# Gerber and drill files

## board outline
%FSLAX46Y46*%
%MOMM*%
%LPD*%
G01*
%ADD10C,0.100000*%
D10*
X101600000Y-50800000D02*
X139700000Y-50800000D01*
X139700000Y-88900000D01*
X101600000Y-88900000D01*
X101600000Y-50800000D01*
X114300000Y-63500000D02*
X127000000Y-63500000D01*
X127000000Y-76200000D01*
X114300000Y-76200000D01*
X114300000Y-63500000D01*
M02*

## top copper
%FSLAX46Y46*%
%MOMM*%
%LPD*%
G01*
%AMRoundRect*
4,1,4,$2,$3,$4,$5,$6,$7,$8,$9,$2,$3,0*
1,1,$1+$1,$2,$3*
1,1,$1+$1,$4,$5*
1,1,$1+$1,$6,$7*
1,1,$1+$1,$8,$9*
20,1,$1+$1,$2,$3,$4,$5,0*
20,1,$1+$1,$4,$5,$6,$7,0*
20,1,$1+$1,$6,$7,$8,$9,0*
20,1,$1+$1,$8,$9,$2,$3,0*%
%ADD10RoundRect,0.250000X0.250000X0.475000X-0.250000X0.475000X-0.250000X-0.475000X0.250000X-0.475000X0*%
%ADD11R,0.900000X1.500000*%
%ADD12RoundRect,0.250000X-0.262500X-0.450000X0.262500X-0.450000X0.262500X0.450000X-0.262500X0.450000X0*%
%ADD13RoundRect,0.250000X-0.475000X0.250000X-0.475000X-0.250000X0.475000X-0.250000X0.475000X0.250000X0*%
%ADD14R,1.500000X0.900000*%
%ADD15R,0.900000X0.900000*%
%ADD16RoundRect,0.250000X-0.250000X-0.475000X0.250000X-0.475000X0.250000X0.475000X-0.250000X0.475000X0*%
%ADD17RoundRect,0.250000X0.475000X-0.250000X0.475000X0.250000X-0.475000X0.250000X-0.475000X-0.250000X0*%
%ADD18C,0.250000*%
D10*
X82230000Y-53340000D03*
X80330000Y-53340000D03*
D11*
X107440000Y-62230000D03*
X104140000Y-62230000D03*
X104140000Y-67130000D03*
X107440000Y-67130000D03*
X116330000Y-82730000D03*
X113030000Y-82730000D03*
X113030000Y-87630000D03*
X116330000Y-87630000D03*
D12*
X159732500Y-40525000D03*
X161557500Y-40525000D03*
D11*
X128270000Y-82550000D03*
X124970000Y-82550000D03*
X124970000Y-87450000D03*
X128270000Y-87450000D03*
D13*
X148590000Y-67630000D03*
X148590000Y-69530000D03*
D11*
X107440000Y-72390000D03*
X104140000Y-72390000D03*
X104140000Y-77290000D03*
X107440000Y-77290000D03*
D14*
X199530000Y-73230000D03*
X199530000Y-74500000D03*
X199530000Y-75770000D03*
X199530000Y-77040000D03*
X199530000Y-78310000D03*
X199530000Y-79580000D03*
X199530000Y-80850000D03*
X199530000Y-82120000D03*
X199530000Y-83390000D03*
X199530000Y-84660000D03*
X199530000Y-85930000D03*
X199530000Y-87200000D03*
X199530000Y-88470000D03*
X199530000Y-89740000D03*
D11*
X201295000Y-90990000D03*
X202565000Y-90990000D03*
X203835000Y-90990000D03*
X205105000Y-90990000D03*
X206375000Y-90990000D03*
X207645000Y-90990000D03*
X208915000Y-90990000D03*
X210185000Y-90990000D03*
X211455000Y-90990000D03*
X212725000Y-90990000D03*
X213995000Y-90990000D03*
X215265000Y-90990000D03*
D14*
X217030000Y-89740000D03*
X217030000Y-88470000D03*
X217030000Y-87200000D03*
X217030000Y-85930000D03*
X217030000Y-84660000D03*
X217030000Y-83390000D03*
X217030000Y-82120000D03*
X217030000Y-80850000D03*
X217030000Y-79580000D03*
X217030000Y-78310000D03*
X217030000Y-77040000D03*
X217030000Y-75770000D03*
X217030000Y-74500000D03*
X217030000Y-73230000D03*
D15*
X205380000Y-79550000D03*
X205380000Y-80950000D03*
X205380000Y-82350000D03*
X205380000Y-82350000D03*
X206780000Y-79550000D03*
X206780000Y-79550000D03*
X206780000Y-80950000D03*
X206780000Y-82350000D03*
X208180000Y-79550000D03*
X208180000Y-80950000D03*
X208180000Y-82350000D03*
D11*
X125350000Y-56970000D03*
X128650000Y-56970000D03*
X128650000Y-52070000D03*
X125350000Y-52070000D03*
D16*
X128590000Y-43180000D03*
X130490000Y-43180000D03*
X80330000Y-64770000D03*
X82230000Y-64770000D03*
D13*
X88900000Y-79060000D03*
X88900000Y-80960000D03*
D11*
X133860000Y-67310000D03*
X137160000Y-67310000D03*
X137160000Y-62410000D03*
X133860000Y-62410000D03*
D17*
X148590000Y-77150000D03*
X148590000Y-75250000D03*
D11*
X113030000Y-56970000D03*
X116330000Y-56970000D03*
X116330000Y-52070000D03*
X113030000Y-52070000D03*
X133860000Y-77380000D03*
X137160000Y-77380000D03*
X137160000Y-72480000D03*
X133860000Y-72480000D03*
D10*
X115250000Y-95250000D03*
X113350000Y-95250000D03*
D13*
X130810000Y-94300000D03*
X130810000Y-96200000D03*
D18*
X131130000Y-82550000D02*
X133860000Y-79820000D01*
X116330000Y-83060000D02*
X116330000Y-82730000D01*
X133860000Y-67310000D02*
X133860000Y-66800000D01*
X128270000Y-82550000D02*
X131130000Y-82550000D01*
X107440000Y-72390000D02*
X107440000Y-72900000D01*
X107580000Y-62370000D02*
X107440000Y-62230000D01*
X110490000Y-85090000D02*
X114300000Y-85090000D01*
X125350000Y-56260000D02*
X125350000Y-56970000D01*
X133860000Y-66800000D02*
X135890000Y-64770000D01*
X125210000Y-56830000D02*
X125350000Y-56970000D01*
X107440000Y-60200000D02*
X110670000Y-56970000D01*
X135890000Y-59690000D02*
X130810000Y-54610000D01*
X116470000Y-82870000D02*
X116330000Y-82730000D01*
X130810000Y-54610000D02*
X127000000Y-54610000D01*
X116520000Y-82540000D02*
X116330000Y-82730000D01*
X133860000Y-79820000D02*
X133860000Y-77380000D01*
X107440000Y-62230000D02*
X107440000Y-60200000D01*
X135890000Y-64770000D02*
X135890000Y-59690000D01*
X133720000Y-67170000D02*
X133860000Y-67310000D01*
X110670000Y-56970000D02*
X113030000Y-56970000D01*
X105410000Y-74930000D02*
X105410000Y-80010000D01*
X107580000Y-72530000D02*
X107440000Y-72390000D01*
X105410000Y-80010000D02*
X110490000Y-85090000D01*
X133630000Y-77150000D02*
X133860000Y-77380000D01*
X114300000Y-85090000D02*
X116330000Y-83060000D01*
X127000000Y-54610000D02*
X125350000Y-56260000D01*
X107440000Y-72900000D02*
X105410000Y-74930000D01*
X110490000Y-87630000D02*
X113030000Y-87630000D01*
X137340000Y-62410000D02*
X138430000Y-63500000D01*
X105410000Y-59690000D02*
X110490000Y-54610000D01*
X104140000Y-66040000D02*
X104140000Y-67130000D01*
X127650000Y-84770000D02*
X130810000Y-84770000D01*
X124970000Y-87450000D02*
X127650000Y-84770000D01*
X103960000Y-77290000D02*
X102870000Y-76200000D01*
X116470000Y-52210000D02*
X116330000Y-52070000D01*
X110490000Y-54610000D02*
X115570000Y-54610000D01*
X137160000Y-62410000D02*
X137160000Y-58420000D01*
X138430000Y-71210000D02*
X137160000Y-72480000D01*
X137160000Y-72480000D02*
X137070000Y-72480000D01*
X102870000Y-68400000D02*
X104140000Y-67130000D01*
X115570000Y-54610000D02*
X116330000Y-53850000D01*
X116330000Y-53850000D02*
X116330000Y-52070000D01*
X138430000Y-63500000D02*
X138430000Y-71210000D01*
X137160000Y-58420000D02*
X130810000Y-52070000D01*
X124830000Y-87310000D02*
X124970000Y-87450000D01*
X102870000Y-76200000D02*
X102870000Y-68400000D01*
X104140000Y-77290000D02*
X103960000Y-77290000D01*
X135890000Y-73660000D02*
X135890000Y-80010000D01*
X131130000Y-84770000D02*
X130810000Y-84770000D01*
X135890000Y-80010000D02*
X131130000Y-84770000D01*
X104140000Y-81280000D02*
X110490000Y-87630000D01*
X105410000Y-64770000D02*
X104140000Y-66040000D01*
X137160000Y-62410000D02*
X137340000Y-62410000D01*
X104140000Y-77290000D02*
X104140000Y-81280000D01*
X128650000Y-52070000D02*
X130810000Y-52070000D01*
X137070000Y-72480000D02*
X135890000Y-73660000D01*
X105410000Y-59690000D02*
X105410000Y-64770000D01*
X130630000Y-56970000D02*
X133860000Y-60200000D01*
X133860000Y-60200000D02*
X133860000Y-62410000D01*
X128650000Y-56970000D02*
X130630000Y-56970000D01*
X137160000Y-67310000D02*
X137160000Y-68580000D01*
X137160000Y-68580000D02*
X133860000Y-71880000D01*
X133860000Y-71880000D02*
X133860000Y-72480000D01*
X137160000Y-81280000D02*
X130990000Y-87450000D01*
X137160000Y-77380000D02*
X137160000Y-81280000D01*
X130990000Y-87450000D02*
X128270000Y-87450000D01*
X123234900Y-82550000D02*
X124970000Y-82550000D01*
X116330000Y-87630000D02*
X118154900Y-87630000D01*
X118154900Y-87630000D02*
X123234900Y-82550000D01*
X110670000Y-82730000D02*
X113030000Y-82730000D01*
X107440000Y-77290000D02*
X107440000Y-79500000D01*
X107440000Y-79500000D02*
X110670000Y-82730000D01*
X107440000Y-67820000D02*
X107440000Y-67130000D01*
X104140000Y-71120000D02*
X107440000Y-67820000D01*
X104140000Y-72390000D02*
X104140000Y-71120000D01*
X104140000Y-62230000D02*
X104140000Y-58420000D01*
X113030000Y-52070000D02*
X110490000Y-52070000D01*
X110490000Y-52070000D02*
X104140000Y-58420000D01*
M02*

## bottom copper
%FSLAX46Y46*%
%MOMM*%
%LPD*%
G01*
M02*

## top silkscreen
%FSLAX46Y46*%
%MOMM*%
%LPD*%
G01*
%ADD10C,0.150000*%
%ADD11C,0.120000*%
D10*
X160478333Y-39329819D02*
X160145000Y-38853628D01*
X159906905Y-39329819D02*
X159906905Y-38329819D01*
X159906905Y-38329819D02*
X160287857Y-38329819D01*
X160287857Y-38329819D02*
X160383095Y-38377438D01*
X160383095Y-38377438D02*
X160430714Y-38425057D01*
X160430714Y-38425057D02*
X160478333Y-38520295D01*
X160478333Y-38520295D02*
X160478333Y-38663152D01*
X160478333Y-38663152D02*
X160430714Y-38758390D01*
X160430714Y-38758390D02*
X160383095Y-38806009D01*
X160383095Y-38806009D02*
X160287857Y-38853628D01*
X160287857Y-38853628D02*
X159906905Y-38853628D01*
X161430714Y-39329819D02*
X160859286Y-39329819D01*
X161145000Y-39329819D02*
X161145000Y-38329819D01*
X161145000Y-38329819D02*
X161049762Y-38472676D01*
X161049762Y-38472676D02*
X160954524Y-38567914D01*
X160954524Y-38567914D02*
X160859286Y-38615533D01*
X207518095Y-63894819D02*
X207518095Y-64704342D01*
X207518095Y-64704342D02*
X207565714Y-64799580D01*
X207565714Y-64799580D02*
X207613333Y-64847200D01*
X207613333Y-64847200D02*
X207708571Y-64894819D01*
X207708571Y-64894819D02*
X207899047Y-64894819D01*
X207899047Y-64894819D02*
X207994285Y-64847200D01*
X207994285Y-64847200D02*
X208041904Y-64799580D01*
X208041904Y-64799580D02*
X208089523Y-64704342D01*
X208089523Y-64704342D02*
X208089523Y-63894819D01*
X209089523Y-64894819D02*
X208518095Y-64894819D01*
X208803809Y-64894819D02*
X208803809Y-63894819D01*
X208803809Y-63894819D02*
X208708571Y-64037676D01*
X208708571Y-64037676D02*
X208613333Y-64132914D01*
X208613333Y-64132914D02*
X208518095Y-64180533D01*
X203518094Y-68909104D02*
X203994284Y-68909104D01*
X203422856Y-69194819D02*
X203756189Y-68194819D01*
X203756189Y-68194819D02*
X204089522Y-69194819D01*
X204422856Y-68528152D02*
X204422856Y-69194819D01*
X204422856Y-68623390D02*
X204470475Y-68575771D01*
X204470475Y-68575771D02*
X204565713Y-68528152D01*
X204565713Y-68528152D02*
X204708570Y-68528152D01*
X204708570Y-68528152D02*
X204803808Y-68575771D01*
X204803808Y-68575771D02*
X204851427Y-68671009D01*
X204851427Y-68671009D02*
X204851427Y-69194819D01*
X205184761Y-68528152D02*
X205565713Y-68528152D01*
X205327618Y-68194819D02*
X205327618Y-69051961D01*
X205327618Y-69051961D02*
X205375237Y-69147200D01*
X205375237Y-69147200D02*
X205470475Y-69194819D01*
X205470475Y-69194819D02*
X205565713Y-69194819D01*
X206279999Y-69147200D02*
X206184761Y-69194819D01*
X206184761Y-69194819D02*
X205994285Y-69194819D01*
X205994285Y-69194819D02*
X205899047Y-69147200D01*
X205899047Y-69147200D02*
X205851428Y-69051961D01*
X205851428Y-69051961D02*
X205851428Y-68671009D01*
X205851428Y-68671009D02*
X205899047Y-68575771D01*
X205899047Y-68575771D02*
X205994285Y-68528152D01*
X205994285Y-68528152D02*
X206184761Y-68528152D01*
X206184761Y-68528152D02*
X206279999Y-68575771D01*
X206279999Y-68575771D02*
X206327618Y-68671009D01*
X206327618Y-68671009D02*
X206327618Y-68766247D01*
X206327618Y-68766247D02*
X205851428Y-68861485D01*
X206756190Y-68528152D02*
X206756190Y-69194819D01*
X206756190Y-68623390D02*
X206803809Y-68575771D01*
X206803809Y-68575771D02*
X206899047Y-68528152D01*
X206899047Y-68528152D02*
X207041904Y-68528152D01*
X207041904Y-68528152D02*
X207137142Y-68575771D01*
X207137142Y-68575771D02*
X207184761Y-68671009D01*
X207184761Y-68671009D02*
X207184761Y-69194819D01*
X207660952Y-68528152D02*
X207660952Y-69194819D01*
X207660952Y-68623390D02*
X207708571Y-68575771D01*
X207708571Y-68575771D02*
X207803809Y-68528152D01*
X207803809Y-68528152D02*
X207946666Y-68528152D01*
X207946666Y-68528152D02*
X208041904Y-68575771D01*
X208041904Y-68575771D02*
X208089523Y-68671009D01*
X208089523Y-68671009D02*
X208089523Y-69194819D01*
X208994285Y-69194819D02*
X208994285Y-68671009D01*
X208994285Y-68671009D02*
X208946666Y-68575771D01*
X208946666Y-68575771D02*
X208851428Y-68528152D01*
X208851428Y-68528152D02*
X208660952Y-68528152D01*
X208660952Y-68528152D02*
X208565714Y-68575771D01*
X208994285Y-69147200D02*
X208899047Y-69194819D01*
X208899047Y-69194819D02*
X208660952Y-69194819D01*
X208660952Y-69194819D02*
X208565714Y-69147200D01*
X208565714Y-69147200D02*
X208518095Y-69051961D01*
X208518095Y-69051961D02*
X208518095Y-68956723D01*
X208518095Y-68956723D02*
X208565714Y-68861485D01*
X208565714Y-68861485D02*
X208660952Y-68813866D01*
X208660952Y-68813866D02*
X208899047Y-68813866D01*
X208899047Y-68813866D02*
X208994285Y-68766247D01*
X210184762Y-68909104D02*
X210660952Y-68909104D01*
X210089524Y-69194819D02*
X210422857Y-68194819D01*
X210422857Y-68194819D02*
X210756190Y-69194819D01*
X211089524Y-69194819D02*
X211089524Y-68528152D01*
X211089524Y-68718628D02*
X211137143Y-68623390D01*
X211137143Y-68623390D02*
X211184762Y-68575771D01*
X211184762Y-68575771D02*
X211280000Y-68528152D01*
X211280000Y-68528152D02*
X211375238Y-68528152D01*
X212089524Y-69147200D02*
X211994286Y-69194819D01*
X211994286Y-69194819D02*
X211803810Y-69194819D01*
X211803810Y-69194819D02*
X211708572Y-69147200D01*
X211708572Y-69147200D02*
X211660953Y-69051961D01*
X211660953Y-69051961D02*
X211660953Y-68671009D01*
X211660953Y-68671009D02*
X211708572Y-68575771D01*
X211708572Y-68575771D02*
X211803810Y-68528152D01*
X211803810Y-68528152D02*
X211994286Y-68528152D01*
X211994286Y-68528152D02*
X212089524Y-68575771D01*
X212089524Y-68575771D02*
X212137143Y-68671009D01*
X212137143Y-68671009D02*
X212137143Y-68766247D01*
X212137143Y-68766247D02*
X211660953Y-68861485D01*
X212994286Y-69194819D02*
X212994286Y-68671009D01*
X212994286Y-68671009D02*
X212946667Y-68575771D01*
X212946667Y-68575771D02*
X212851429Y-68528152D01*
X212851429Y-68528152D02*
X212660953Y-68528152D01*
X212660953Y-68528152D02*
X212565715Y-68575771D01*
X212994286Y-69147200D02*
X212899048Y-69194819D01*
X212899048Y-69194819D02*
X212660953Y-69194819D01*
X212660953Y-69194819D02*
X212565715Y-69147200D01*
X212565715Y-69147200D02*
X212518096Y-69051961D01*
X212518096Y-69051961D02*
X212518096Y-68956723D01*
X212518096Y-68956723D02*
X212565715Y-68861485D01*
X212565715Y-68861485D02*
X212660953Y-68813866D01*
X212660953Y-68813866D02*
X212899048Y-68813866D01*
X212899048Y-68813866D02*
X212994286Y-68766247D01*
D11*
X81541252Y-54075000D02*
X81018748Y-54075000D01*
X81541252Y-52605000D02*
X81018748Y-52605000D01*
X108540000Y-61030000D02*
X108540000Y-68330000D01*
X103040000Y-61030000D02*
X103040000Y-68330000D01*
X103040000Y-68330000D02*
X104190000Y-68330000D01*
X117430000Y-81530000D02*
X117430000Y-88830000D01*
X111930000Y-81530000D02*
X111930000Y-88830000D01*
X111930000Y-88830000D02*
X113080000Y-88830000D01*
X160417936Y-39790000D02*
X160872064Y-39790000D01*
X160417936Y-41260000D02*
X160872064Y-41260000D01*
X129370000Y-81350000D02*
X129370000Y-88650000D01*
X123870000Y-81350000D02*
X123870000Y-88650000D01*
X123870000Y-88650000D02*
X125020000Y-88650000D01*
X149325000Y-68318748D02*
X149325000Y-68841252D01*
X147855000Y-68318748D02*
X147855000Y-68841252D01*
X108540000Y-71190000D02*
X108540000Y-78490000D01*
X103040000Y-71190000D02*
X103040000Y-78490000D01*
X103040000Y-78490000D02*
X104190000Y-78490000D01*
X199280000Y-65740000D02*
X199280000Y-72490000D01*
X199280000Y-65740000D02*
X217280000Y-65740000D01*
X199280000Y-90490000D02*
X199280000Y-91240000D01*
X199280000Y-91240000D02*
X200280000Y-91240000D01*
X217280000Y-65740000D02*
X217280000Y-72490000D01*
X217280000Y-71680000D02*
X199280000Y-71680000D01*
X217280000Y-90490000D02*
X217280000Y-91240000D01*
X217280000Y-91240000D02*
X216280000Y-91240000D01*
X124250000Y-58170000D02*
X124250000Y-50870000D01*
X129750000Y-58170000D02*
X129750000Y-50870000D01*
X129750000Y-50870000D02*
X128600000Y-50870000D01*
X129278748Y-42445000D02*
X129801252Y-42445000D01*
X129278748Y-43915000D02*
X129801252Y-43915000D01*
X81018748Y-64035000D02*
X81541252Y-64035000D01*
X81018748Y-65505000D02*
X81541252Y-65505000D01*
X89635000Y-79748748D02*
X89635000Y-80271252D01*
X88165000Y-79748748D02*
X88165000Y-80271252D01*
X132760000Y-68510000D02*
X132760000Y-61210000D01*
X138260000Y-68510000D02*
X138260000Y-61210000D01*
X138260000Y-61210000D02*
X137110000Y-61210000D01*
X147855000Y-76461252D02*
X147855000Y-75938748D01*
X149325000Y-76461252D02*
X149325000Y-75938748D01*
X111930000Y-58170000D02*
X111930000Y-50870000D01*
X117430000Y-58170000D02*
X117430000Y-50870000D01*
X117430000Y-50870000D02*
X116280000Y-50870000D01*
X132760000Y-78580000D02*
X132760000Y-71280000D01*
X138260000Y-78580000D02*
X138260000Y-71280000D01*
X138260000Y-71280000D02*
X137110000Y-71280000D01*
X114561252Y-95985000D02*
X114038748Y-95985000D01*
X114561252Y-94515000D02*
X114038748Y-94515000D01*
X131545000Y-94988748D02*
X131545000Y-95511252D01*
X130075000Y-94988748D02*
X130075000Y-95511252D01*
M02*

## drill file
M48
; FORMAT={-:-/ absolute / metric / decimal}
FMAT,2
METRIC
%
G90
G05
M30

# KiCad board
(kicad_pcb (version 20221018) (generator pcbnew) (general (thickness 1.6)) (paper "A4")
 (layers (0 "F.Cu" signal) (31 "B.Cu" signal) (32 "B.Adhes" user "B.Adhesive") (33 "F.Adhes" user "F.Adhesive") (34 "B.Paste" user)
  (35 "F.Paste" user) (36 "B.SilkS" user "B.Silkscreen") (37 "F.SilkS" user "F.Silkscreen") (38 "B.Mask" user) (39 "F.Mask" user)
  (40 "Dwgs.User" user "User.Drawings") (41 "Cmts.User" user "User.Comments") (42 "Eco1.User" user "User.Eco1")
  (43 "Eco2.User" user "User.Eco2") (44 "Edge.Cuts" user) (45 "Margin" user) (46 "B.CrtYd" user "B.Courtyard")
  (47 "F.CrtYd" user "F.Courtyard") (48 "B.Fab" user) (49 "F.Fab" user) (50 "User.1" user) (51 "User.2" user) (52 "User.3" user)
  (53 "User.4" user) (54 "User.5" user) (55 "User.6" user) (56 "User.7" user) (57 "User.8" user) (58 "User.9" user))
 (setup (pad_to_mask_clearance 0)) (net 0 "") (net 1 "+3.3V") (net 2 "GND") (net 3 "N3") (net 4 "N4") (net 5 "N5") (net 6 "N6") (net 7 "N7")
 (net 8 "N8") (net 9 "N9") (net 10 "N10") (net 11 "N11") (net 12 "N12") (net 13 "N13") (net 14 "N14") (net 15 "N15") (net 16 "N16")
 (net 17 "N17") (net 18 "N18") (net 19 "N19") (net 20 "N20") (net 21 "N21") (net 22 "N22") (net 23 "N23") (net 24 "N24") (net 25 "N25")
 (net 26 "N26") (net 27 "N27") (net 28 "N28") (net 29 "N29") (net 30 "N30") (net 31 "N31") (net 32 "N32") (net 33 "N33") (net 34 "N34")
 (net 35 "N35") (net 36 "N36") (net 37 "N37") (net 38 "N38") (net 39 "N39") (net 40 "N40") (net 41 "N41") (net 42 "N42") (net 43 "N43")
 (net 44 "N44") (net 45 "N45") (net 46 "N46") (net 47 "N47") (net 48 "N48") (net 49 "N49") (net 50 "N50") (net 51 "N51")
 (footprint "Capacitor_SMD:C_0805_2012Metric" (layer "F.Cu") (at 81.28 53.34 180)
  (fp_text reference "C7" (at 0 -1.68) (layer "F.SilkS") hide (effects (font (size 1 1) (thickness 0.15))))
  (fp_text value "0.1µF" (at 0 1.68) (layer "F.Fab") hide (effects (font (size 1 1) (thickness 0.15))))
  (fp_line (start -0.261252 -0.735) (end 0.261252 -0.735) (stroke (width 0.12) (type solid)) (layer "F.SilkS"))
  (fp_line (start -0.261252 0.735) (end 0.261252 0.735) (stroke (width 0.12) (type solid)) (layer "F.SilkS"))
  (pad "1" smd roundrect (at -0.95 0 180) (size 1 1.45) (layers "F.Cu" "F.Paste" "F.Mask") (roundrect_rratio 0.25) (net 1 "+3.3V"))
  (pad "2" smd roundrect (at 0.95 0 180) (size 1 1.45) (layers "F.Cu" "F.Paste" "F.Mask") (roundrect_rratio 0.25) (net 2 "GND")))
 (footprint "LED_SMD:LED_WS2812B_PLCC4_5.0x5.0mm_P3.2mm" (layer "F.Cu") (at 105.79 64.68 -90)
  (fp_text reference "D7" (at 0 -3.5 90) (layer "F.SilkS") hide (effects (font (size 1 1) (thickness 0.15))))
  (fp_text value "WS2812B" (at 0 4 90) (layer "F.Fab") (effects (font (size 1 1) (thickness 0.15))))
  (fp_line (start -3.65 -2.75) (end 3.65 -2.75) (stroke (width 0.12) (type solid)) (layer "F.SilkS"))
  (fp_line (start -3.65 2.75) (end 3.65 2.75) (stroke (width 0.12) (type solid)) (layer "F.SilkS"))
  (fp_line (start 3.65 2.75) (end 3.65 1.6) (stroke (width 0.12) (type solid)) (layer "F.SilkS"))
  (pad "1" smd rect (at -2.45 -1.65 270) (size 1.5 0.9) (layers "F.Cu" "F.Paste" "F.Mask") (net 1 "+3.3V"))
  (pad "2" smd rect (at -2.45 1.65 270) (size 1.5 0.9) (layers "F.Cu" "F.Paste" "F.Mask") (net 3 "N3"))
  (pad "3" smd rect (at 2.45 1.65 270) (size 1.5 0.9) (layers "F.Cu" "F.Paste" "F.Mask") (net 2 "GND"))
  (pad "4" smd rect (at 2.45 -1.65 270) (size 1.5 0.9) (layers "F.Cu" "F.Paste" "F.Mask") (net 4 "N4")))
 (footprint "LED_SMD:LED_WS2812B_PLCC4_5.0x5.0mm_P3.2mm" (layer "F.Cu") (at 114.68 85.18 -90)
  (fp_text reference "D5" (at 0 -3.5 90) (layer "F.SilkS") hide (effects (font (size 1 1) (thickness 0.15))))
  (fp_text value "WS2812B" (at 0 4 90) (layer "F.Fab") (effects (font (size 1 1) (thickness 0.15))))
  (fp_line (start -3.65 -2.75) (end 3.65 -2.75) (stroke (width 0.12) (type solid)) (layer "F.SilkS"))
  (fp_line (start -3.65 2.75) (end 3.65 2.75) (stroke (width 0.12) (type solid)) (layer "F.SilkS"))
  (fp_line (start 3.65 2.75) (end 3.65 1.6) (stroke (width 0.12) (type solid)) (layer "F.SilkS"))
  (pad "1" smd rect (at -2.45 -1.65 270) (size 1.5 0.9) (layers "F.Cu" "F.Paste" "F.Mask") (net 1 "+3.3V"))
  (pad "2" smd rect (at -2.45 1.65 270) (size 1.5 0.9) (layers "F.Cu" "F.Paste" "F.Mask") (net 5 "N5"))
  (pad "3" smd rect (at 2.45 1.65 270) (size 1.5 0.9) (layers "F.Cu" "F.Paste" "F.Mask") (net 2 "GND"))
  (pad "4" smd rect (at 2.45 -1.65 270) (size 1.5 0.9) (layers "F.Cu" "F.Paste" "F.Mask") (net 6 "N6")))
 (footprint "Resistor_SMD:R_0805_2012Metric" (layer "F.Cu") (at 160.645 40.525)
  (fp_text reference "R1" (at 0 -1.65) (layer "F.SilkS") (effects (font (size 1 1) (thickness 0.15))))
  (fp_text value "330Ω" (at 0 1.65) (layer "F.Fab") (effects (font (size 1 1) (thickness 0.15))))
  (fp_line (start -0.227064 -0.735) (end 0.227064 -0.735) (stroke (width 0.12) (type solid)) (layer "F.SilkS"))
  (fp_line (start -0.227064 0.735) (end 0.227064 0.735) (stroke (width 0.12) (type solid)) (layer "F.SilkS"))
  (pad "1" smd roundrect (at -0.9125 0) (size 1.025 1.4) (layers "F.Cu" "F.Paste" "F.Mask") (roundrect_rratio 0.243902) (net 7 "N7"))
  (pad "2" smd roundrect (at 0.9125 0) (size 1.025 1.4) (layers "F.Cu" "F.Paste" "F.Mask") (roundrect_rratio 0.243902) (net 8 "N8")))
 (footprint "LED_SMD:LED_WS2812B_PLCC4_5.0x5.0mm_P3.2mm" (layer "F.Cu") (at 126.62 85 -90)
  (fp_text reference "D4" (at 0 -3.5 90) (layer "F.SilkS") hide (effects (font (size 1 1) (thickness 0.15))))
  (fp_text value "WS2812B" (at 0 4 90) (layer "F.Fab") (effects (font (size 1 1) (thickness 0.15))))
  (fp_line (start -3.65 -2.75) (end 3.65 -2.75) (stroke (width 0.12) (type solid)) (layer "F.SilkS"))
  (fp_line (start -3.65 2.75) (end 3.65 2.75) (stroke (width 0.12) (type solid)) (layer "F.SilkS"))
  (fp_line (start 3.65 2.75) (end 3.65 1.6) (stroke (width 0.12) (type solid)) (layer "F.SilkS"))
  (pad "1" smd rect (at -2.45 -1.65 270) (size 1.5 0.9) (layers "F.Cu" "F.Paste" "F.Mask") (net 1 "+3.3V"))
  (pad "2" smd rect (at -2.45 1.65 270) (size 1.5 0.9) (layers "F.Cu" "F.Paste" "F.Mask") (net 6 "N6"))
  (pad "3" smd rect (at 2.45 1.65 270) (size 1.5 0.9) (layers "F.Cu" "F.Paste" "F.Mask") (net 2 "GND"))
  (pad "4" smd rect (at 2.45 -1.65 270) (size 1.5 0.9) (layers "F.Cu" "F.Paste" "F.Mask") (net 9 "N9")))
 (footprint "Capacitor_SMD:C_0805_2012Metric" (layer "F.Cu") (at 148.59 68.58 -90)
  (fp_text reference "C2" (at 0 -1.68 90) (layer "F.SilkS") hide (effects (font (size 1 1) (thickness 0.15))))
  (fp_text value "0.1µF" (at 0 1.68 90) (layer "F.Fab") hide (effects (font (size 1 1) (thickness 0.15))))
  (fp_line (start -0.261252 -0.735) (end 0.261252 -0.735) (stroke (width 0.12) (type solid)) (layer "F.SilkS"))
  (fp_line (start -0.261252 0.735) (end 0.261252 0.735) (stroke (width 0.12) (type solid)) (layer "F.SilkS"))
  (pad "1" smd roundrect (at -0.95 0 270) (size 1 1.45) (layers "F.Cu" "F.Paste" "F.Mask") (roundrect_rratio 0.25) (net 1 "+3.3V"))
  (pad "2" smd roundrect (at 0.95 0 270) (size 1 1.45) (layers "F.Cu" "F.Paste" "F.Mask") (roundrect_rratio 0.25) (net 2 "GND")))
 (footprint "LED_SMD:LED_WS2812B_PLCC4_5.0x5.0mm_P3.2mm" (layer "F.Cu") (at 105.79 74.84 -90)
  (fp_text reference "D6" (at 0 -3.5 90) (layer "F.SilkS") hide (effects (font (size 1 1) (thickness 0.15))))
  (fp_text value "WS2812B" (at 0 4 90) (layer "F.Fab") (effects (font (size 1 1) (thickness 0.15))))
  (fp_line (start -3.65 -2.75) (end 3.65 -2.75) (stroke (width 0.12) (type solid)) (layer "F.SilkS"))
  (fp_line (start -3.65 2.75) (end 3.65 2.75) (stroke (width 0.12) (type solid)) (layer "F.SilkS"))
  (fp_line (start 3.65 2.75) (end 3.65 1.6) (stroke (width 0.12) (type solid)) (layer "F.SilkS"))
  (pad "1" smd rect (at -2.45 -1.65 270) (size 1.5 0.9) (layers "F.Cu" "F.Paste" "F.Mask") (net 1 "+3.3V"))
  (pad "2" smd rect (at -2.45 1.65 270) (size 1.5 0.9) (layers "F.Cu" "F.Paste" "F.Mask") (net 4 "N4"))
  (pad "3" smd rect (at 2.45 1.65 270) (size 1.5 0.9) (layers "F.Cu" "F.Paste" "F.Mask") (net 2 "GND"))
  (pad "4" smd rect (at 2.45 -1.65 270) (size 1.5 0.9) (layers "F.Cu" "F.Paste" "F.Mask") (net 5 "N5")))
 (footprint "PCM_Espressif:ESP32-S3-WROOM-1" (layer "F.Cu") (at 208.28 81.49)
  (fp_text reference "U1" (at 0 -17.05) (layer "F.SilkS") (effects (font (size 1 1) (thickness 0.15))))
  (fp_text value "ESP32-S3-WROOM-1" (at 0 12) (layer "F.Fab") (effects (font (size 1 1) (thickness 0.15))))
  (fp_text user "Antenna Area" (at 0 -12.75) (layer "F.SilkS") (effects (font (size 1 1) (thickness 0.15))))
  (fp_line (start -9 -15.75) (end -9 -9) (stroke (width 0.12) (type solid)) (layer "F.SilkS"))
  (fp_line (start -9 -15.75) (end 9 -15.75) (stroke (width 0.12) (type solid)) (layer "F.SilkS"))
  (fp_line (start -9 9) (end -9 9.75) (stroke (width 0.12) (type solid)) (layer "F.SilkS"))
  (fp_line (start -9 9.75) (end -8 9.75) (stroke (width 0.12) (type solid)) (layer "F.SilkS"))
  (fp_line (start 9 -15.75) (end 9 -9) (stroke (width 0.12) (type solid)) (layer "F.SilkS"))
  (fp_line (start 9 -9.81) (end -9 -9.81) (stroke (width 0.12) (type solid)) (layer "F.SilkS"))
  (fp_line (start 9 9) (end 9 9.75) (stroke (width 0.12) (type solid)) (layer "F.SilkS"))
  (fp_line (start 9 9.75) (end 8 9.75) (stroke (width 0.12) (type solid)) (layer "F.SilkS"))
  (pad "1" smd rect (at -8.75 -8.26) (size 1.5 0.9) (layers "F.Cu" "F.Paste" "F.Mask") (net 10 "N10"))
  (pad "2" smd rect (at -8.75 -6.99) (size 1.5 0.9) (layers "F.Cu" "F.Paste" "F.Mask") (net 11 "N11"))
  (pad "3" smd rect (at -8.75 -5.72) (size 1.5 0.9) (layers "F.Cu" "F.Paste" "F.Mask") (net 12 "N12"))
  (pad "4" smd rect (at -8.75 -4.45) (size 1.5 0.9) (layers "F.Cu" "F.Paste" "F.Mask") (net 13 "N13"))
  (pad "5" smd rect (at -8.75 -3.18) (size 1.5 0.9) (layers "F.Cu" "F.Paste" "F.Mask") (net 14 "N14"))
  (pad "6" smd rect (at -8.75 -1.91) (size 1.5 0.9) (layers "F.Cu" "F.Paste" "F.Mask") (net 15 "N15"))
  (pad "7" smd rect (at -8.75 -0.64) (size 1.5 0.9) (layers "F.Cu" "F.Paste" "F.Mask") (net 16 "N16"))
  (pad "8" smd rect (at -8.75 0.63) (size 1.5 0.9) (layers "F.Cu" "F.Paste" "F.Mask") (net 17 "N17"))
  (pad "9" smd rect (at -8.75 1.9) (size 1.5 0.9) (layers "F.Cu" "F.Paste" "F.Mask") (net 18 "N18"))
  (pad "10" smd rect (at -8.75 3.17) (size 1.5 0.9) (layers "F.Cu" "F.Paste" "F.Mask") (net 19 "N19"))
  (pad "11" smd rect (at -8.75 4.44) (size 1.5 0.9) (layers "F.Cu" "F.Paste" "F.Mask") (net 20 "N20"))
  (pad "12" smd rect (at -8.75 5.71) (size 1.5 0.9) (layers "F.Cu" "F.Paste" "F.Mask") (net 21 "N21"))
  (pad "13" smd rect (at -8.75 6.98) (size 1.5 0.9) (layers "F.Cu" "F.Paste" "F.Mask") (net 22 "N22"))
  (pad "14" smd rect (at -8.75 8.25) (size 1.5 0.9) (layers "F.Cu" "F.Paste" "F.Mask") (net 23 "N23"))
  (pad "15" smd rect (at -6.985 9.5 90) (size 1.5 0.9) (layers "F.Cu" "F.Paste" "F.Mask") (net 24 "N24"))
  (pad "16" smd rect (at -5.715 9.5 90) (size 1.5 0.9) (layers "F.Cu" "F.Paste" "F.Mask") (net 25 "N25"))
  (pad "17" smd rect (at -4.445 9.5 90) (size 1.5 0.9) (layers "F.Cu" "F.Paste" "F.Mask") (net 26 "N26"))
  (pad "18" smd rect (at -3.175 9.5 90) (size 1.5 0.9) (layers "F.Cu" "F.Paste" "F.Mask") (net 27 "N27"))
  (pad "19" smd rect (at -1.905 9.5 90) (size 1.5 0.9) (layers "F.Cu" "F.Paste" "F.Mask") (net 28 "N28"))
  (pad "20" smd rect (at -0.635 9.5 90) (size 1.5 0.9) (layers "F.Cu" "F.Paste" "F.Mask") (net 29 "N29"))
  (pad "21" smd rect (at 0.635 9.5 90) (size 1.5 0.9) (layers "F.Cu" "F.Paste" "F.Mask") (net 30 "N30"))
  (pad "22" smd rect (at 1.905 9.5 90) (size 1.5 0.9) (layers "F.Cu" "F.Paste" "F.Mask") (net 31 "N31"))
  (pad "23" smd rect (at 3.175 9.5 90) (size 1.5 0.9) (layers "F.Cu" "F.Paste" "F.Mask") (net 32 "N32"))
  (pad "24" smd rect (at 4.445 9.5 90) (size 1.5 0.9) (layers "F.Cu" "F.Paste" "F.Mask") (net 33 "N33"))
  (pad "25" smd rect (at 5.715 9.5 90) (size 1.5 0.9) (layers "F.Cu" "F.Paste" "F.Mask") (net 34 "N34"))
  (pad "26" smd rect (at 6.985 9.5 90) (size 1.5 0.9) (layers "F.Cu" "F.Paste" "F.Mask") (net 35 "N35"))
  (pad "27" smd rect (at 8.75 8.25 180) (size 1.5 0.9) (layers "F.Cu" "F.Paste" "F.Mask") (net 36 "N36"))
  (pad "28" smd rect (at 8.75 6.98 180) (size 1.5 0.9) (layers "F.Cu" "F.Paste" "F.Mask") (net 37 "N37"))
  (pad "29" smd rect (at 8.75 5.71 180) (size 1.5 0.9) (layers "F.Cu" "F.Paste" "F.Mask") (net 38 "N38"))
  (pad "30" smd rect (at 8.75 4.44 180) (size 1.5 0.9) (layers "F.Cu" "F.Paste" "F.Mask") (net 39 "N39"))
  (pad "31" smd rect (at 8.75 3.17 180) (size 1.5 0.9) (layers "F.Cu" "F.Paste" "F.Mask") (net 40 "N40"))
  (pad "32" smd rect (at 8.75 1.9 180) (size 1.5 0.9) (layers "F.Cu" "F.Paste" "F.Mask") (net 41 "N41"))
  (pad "33" smd rect (at 8.75 0.63 180) (size 1.5 0.9) (layers "F.Cu" "F.Paste" "F.Mask") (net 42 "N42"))
  (pad "34" smd rect (at 8.75 -0.64 180) (size 1.5 0.9) (layers "F.Cu" "F.Paste" "F.Mask") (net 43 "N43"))
  (pad "35" smd rect (at 8.75 -1.91 180) (size 1.5 0.9) (layers "F.Cu" "F.Paste" "F.Mask") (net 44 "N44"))
  (pad "36" smd rect (at 8.75 -3.18 180) (size 1.5 0.9) (layers "F.Cu" "F.Paste" "F.Mask") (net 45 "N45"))
  (pad "37" smd rect (at 8.75 -4.45 180) (size 1.5 0.9) (layers "F.Cu" "F.Paste" "F.Mask") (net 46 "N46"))
  (pad "38" smd rect (at 8.75 -5.72 180) (size 1.5 0.9) (layers "F.Cu" "F.Paste" "F.Mask") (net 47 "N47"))
  (pad "39" smd rect (at 8.75 -6.99 180) (size 1.5 0.9) (layers "F.Cu" "F.Paste" "F.Mask") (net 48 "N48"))
  (pad "40" smd rect (at 8.75 -8.26 180) (size 1.5 0.9) (layers "F.Cu" "F.Paste" "F.Mask") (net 10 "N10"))
  (pad "41" smd rect (at -2.9 -1.94 180) (size 0.9 0.9) (layers "F.Cu" "F.Paste" "F.Mask") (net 10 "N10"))
  (pad "41" smd rect (at -2.9 -0.54 180) (size 0.9 0.9) (layers "F.Cu" "F.Paste" "F.Mask") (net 10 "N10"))
  (pad "41" smd rect (at -2.9 0.86 180) (size 0.9 0.9) (layers "F.Cu" "F.Paste" "F.Mask") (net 10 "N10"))
  (pad "41" smd rect (at -2.9 0.86 180) (size 0.9 0.9) (layers "F.Cu" "F.Paste" "F.Mask") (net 10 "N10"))
  (pad "41" smd rect (at -1.5 -1.94 180) (size 0.9 0.9) (layers "F.Cu" "F.Paste" "F.Mask") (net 10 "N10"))
  (pad "41" smd rect (at -1.5 -1.94 180) (size 0.9 0.9) (layers "F.Cu" "F.Paste" "F.Mask") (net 10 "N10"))
  (pad "41" smd rect (at -1.5 -0.54 180) (size 0.9 0.9) (layers "F.Cu" "F.Paste" "F.Mask") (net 10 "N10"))
  (pad "41" smd rect (at -1.5 0.86 180) (size 0.9 0.9) (layers "F.Cu" "F.Paste" "F.Mask") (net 10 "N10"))
  (pad "41" smd rect (at -0.1 -1.94 180) (size 0.9 0.9) (layers "F.Cu" "F.Paste" "F.Mask") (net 10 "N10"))
  (pad "41" smd rect (at -0.1 -0.54 180) (size 0.9 0.9) (layers "F.Cu" "F.Paste" "F.Mask") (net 10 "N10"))
  (pad "41" smd rect (at -0.1 0.86 180) (size 0.9 0.9) (layers "F.Cu" "F.Paste" "F.Mask") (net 10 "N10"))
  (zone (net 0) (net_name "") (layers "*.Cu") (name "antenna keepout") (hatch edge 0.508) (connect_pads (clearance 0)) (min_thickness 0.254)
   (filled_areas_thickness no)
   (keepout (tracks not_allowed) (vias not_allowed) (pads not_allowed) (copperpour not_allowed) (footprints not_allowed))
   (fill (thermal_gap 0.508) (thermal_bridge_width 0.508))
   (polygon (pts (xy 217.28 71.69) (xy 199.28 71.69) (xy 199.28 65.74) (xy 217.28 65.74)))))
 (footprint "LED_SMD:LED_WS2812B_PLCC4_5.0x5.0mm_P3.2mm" (layer "F.Cu") (at 127 54.52 90)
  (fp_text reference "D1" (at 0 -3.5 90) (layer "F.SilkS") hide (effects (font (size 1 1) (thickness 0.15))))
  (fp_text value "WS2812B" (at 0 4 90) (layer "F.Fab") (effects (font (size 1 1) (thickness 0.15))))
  (fp_line (start -3.65 -2.75) (end 3.65 -2.75) (stroke (width 0.12) (type solid)) (layer "F.SilkS"))
  (fp_line (start -3.65 2.75) (end 3.65 2.75) (stroke (width 0.12) (type solid)) (layer "F.SilkS"))
  (fp_line (start 3.65 2.75) (end 3.65 1.6) (stroke (width 0.12) (type solid)) (layer "F.SilkS"))
  (pad "1" smd rect (at -2.45 -1.65 90) (size 1.5 0.9) (layers "F.Cu" "F.Paste" "F.Mask") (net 1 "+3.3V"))
  (pad "2" smd rect (at -2.45 1.65 90) (size 1.5 0.9) (layers "F.Cu" "F.Paste" "F.Mask") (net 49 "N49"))
  (pad "3" smd rect (at 2.45 1.65 90) (size 1.5 0.9) (layers "F.Cu" "F.Paste" "F.Mask") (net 2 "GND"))
  (pad "4" smd rect (at 2.45 -1.65 90) (size 1.5 0.9) (layers "F.Cu" "F.Paste" "F.Mask") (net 8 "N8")))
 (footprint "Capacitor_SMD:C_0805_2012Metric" (layer "F.Cu") (at 129.54 43.18)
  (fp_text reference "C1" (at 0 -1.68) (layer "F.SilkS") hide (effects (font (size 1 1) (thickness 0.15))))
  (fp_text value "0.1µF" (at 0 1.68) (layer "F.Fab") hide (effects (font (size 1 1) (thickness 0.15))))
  (fp_line (start -0.261252 -0.735) (end 0.261252 -0.735) (stroke (width 0.12) (type solid)) (layer "F.SilkS"))
  (fp_line (start -0.261252 0.735) (end 0.261252 0.735) (stroke (width 0.12) (type solid)) (layer "F.SilkS"))
  (pad "1" smd roundrect (at -0.95 0) (size 1 1.45) (layers "F.Cu" "F.Paste" "F.Mask") (roundrect_rratio 0.25) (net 1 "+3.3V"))
  (pad "2" smd roundrect (at 0.95 0) (size 1 1.45) (layers "F.Cu" "F.Paste" "F.Mask") (roundrect_rratio 0.25) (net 2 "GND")))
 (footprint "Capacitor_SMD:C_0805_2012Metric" (layer "F.Cu") (at 81.28 64.77)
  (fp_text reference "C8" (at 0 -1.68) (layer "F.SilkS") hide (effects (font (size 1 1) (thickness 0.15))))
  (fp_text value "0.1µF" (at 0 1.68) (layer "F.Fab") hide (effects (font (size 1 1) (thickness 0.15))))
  (fp_line (start -0.261252 -0.735) (end 0.261252 -0.735) (stroke (width 0.12) (type solid)) (layer "F.SilkS"))
  (fp_line (start -0.261252 0.735) (end 0.261252 0.735) (stroke (width 0.12) (type solid)) (layer "F.SilkS"))
  (pad "1" smd roundrect (at -0.95 0) (size 1 1.45) (layers "F.Cu" "F.Paste" "F.Mask") (roundrect_rratio 0.25) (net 1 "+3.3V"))
  (pad "2" smd roundrect (at 0.95 0) (size 1 1.45) (layers "F.Cu" "F.Paste" "F.Mask") (roundrect_rratio 0.25) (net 2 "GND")))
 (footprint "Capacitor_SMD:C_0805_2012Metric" (layer "F.Cu") (at 88.9 80.01 -90)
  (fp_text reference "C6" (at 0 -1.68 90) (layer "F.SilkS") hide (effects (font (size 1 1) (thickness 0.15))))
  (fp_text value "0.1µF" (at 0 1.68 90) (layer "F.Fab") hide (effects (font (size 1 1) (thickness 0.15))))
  (fp_line (start -0.261252 -0.735) (end 0.261252 -0.735) (stroke (width 0.12) (type solid)) (layer "F.SilkS"))
  (fp_line (start -0.261252 0.735) (end 0.261252 0.735) (stroke (width 0.12) (type solid)) (layer "F.SilkS"))
  (pad "1" smd roundrect (at -0.95 0 270) (size 1 1.45) (layers "F.Cu" "F.Paste" "F.Mask") (roundrect_rratio 0.25) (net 1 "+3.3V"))
  (pad "2" smd roundrect (at 0.95 0 270) (size 1 1.45) (layers "F.Cu" "F.Paste" "F.Mask") (roundrect_rratio 0.25) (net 2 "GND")))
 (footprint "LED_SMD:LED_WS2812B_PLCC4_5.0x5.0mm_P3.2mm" (layer "F.Cu") (at 135.51 64.86 90)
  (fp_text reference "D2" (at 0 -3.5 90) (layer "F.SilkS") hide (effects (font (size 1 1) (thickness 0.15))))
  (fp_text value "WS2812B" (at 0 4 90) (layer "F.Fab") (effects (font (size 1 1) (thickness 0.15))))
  (fp_line (start -3.65 -2.75) (end 3.65 -2.75) (stroke (width 0.12) (type solid)) (layer "F.SilkS"))
  (fp_line (start -3.65 2.75) (end 3.65 2.75) (stroke (width 0.12) (type solid)) (layer "F.SilkS"))
  (fp_line (start 3.65 2.75) (end 3.65 1.6) (stroke (width 0.12) (type solid)) (layer "F.SilkS"))
  (pad "1" smd rect (at -2.45 -1.65 90) (size 1.5 0.9) (layers "F.Cu" "F.Paste" "F.Mask") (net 1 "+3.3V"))
  (pad "2" smd rect (at -2.45 1.65 90) (size 1.5 0.9) (layers "F.Cu" "F.Paste" "F.Mask") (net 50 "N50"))
  (pad "3" smd rect (at 2.45 1.65 90) (size 1.5 0.9) (layers "F.Cu" "F.Paste" "F.Mask") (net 2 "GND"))
  (pad "4" smd rect (at 2.45 -1.65 90) (size 1.5 0.9) (layers "F.Cu" "F.Paste" "F.Mask") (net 49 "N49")))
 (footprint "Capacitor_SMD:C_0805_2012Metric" (layer "F.Cu") (at 148.59 76.2 90)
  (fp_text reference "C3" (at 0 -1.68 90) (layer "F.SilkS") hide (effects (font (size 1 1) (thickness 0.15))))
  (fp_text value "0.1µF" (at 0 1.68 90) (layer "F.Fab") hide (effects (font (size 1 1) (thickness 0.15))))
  (fp_line (start -0.261252 -0.735) (end 0.261252 -0.735) (stroke (width 0.12) (type solid)) (layer "F.SilkS"))
  (fp_line (start -0.261252 0.735) (end 0.261252 0.735) (stroke (width 0.12) (type solid)) (layer "F.SilkS"))
  (pad "1" smd roundrect (at -0.95 0 90) (size 1 1.45) (layers "F.Cu" "F.Paste" "F.Mask") (roundrect_rratio 0.25) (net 1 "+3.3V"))
  (pad "2" smd roundrect (at 0.95 0 90) (size 1 1.45) (layers "F.Cu" "F.Paste" "F.Mask") (roundrect_rratio 0.25) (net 2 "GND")))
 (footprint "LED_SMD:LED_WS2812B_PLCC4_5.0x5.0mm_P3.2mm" (layer "F.Cu") (at 114.68 54.52 90)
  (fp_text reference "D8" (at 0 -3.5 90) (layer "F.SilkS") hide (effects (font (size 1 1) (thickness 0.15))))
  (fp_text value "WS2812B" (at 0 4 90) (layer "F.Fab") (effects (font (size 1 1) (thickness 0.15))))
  (fp_line (start -3.65 -2.75) (end 3.65 -2.75) (stroke (width 0.12) (type solid)) (layer "F.SilkS"))
  (fp_line (start -3.65 2.75) (end 3.65 2.75) (stroke (width 0.12) (type solid)) (layer "F.SilkS"))
  (fp_line (start 3.65 2.75) (end 3.65 1.6) (stroke (width 0.12) (type solid)) (layer "F.SilkS"))
  (pad "1" smd rect (at -2.45 -1.65 90) (size 1.5 0.9) (layers "F.Cu" "F.Paste" "F.Mask") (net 1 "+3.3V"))
  (pad "2" smd rect (at -2.45 1.65 90) (size 1.5 0.9) (layers "F.Cu" "F.Paste" "F.Mask") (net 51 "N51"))
  (pad "3" smd rect (at 2.45 1.65 90) (size 1.5 0.9) (layers "F.Cu" "F.Paste" "F.Mask") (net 2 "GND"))
  (pad "4" smd rect (at 2.45 -1.65 90) (size 1.5 0.9) (layers "F.Cu" "F.Paste" "F.Mask") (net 3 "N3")))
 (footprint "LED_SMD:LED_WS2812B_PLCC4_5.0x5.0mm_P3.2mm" (layer "F.Cu") (at 135.51 74.93 90)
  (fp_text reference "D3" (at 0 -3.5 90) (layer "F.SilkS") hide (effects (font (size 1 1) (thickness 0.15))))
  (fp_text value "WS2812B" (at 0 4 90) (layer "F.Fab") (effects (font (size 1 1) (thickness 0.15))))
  (fp_line (start -3.65 -2.75) (end 3.65 -2.75) (stroke (width 0.12) (type solid)) (layer "F.SilkS"))
  (fp_line (start -3.65 2.75) (end 3.65 2.75) (stroke (width 0.12) (type solid)) (layer "F.SilkS"))
  (fp_line (start 3.65 2.75) (end 3.65 1.6) (stroke (width 0.12) (type solid)) (layer "F.SilkS"))
  (pad "1" smd rect (at -2.45 -1.65 90) (size 1.5 0.9) (layers "F.Cu" "F.Paste" "F.Mask") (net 1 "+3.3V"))
  (pad "2" smd rect (at -2.45 1.65 90) (size 1.5 0.9) (layers "F.Cu" "F.Paste" "F.Mask") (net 9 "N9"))
  (pad "3" smd rect (at 2.45 1.65 90) (size 1.5 0.9) (layers "F.Cu" "F.Paste" "F.Mask") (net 2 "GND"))
  (pad "4" smd rect (at 2.45 -1.65 90) (size 1.5 0.9) (layers "F.Cu" "F.Paste" "F.Mask") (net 50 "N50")))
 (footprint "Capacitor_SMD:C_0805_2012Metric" (layer "F.Cu") (at 114.3 95.25 180)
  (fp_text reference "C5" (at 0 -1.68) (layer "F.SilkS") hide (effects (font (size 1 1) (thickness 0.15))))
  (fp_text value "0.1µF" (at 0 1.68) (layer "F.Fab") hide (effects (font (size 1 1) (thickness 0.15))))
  (fp_line (start -0.261252 -0.735) (end 0.261252 -0.735) (stroke (width 0.12) (type solid)) (layer "F.SilkS"))
  (fp_line (start -0.261252 0.735) (end 0.261252 0.735) (stroke (width 0.12) (type solid)) (layer "F.SilkS"))
  (pad "1" smd roundrect (at -0.95 0 180) (size 1 1.45) (layers "F.Cu" "F.Paste" "F.Mask") (roundrect_rratio 0.25) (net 1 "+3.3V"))
  (pad "2" smd roundrect (at 0.95 0 180) (size 1 1.45) (layers "F.Cu" "F.Paste" "F.Mask") (roundrect_rratio 0.25) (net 2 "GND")))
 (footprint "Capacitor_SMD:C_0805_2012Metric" (layer "F.Cu") (at 130.81 95.25 -90)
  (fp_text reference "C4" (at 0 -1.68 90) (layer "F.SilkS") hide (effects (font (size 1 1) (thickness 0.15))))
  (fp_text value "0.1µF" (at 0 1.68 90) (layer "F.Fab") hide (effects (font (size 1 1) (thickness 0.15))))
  (fp_line (start -0.261252 -0.735) (end 0.261252 -0.735) (stroke (width 0.12) (type solid)) (layer "F.SilkS"))
  (fp_line (start -0.261252 0.735) (end 0.261252 0.735) (stroke (width 0.12) (type solid)) (layer "F.SilkS"))
  (pad "1" smd roundrect (at -0.95 0 270) (size 1 1.45) (layers "F.Cu" "F.Paste" "F.Mask") (roundrect_rratio 0.25) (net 1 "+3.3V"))
  (pad "2" smd roundrect (at 0.95 0 270) (size 1 1.45) (layers "F.Cu" "F.Paste" "F.Mask") (roundrect_rratio 0.25) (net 2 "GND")))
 (gr_rect (start 101.6 50.8) (end 139.7 88.9) (stroke (width 0.1) (type default)) (fill none) (layer "Edge.Cuts"))
 (gr_rect (start 114.3 63.5) (end 127 76.2) (stroke (width 0.1) (type default)) (fill none) (layer "Edge.Cuts"))
 (segment (start 131.13 82.55) (end 133.86 79.82) (width 0.25) (layer "F.Cu") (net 1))
 (segment (start 116.33 83.06) (end 116.33 82.73) (width 0.25) (layer "F.Cu") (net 1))
 (segment (start 133.86 67.31) (end 133.86 66.8) (width 0.25) (layer "F.Cu") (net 1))
 (segment (start 128.27 82.55) (end 131.13 82.55) (width 0.25) (layer "F.Cu") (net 1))
 (segment (start 107.44 72.39) (end 107.44 72.9) (width 0.25) (layer "F.Cu") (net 1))
 (segment (start 107.58 62.37) (end 107.44 62.23) (width 0.25) (layer "F.Cu") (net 1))
 (segment (start 110.49 85.09) (end 114.3 85.09) (width 0.25) (layer "F.Cu") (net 1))
 (segment (start 125.35 56.26) (end 125.35 56.97) (width 0.25) (layer "F.Cu") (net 1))
 (segment (start 133.86 66.8) (end 135.89 64.77) (width 0.25) (layer "F.Cu") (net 1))
 (segment (start 125.21 56.83) (end 125.35 56.97) (width 0.25) (layer "F.Cu") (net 1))
 (segment (start 107.44 60.2) (end 110.67 56.97) (width 0.25) (layer "F.Cu") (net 1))
 (segment (start 135.89 59.69) (end 130.81 54.61) (width 0.25) (layer "F.Cu") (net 1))
 (segment (start 116.47 82.87) (end 116.33 82.73) (width 0.25) (layer "F.Cu") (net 1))
 (segment (start 130.81 54.61) (end 127 54.61) (width 0.25) (layer "F.Cu") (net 1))
 (segment (start 116.52 82.54) (end 116.33 82.73) (width 0.25) (layer "F.Cu") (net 1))
 (segment (start 133.86 79.82) (end 133.86 77.38) (width 0.25) (layer "F.Cu") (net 1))
 (segment (start 107.44 62.23) (end 107.44 60.2) (width 0.25) (layer "F.Cu") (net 1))
 (segment (start 135.89 64.77) (end 135.89 59.69) (width 0.25) (layer "F.Cu") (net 1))
 (segment (start 133.72 67.17) (end 133.86 67.31) (width 0.25) (layer "F.Cu") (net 1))
 (segment (start 110.67 56.97) (end 113.03 56.97) (width 0.25) (layer "F.Cu") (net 1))
 (segment (start 105.41 74.93) (end 105.41 80.01) (width 0.25) (layer "F.Cu") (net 1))
 (segment (start 107.58 72.53) (end 107.44 72.39) (width 0.25) (layer "F.Cu") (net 1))
 (segment (start 105.41 80.01) (end 110.49 85.09) (width 0.25) (layer "F.Cu") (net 1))
 (segment (start 133.63 77.15) (end 133.86 77.38) (width 0.25) (layer "F.Cu") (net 1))
 (segment (start 114.3 85.09) (end 116.33 83.06) (width 0.25) (layer "F.Cu") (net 1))
 (segment (start 127 54.61) (end 125.35 56.26) (width 0.25) (layer "F.Cu") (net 1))
 (segment (start 107.44 72.9) (end 105.41 74.93) (width 0.25) (layer "F.Cu") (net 1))
 (segment (start 110.49 87.63) (end 113.03 87.63) (width 0.25) (layer "F.Cu") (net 2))
 (segment (start 137.34 62.41) (end 138.43 63.5) (width 0.25) (layer "F.Cu") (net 2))
 (segment (start 105.41 59.69) (end 110.49 54.61) (width 0.25) (layer "F.Cu") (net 2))
 (segment (start 104.14 66.04) (end 104.14 67.13) (width 0.25) (layer "F.Cu") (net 2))
 (segment (start 127.65 84.77) (end 130.81 84.77) (width 0.25) (layer "F.Cu") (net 2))
 (segment (start 124.97 87.45) (end 127.65 84.77) (width 0.25) (layer "F.Cu") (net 2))
 (segment (start 103.96 77.29) (end 102.87 76.2) (width 0.25) (layer "F.Cu") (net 2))
 (segment (start 116.47 52.21) (end 116.33 52.07) (width 0.25) (layer "F.Cu") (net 2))
 (segment (start 110.49 54.61) (end 115.57 54.61) (width 0.25) (layer "F.Cu") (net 2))
 (segment (start 137.16 62.41) (end 137.16 58.42) (width 0.25) (layer "F.Cu") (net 2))
 (segment (start 138.43 71.21) (end 137.16 72.48) (width 0.25) (layer "F.Cu") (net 2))
 (segment (start 137.16 72.48) (end 137.07 72.48) (width 0.25) (layer "F.Cu") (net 2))
 (segment (start 102.87 68.4) (end 104.14 67.13) (width 0.25) (layer "F.Cu") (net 2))
 (segment (start 115.57 54.61) (end 116.33 53.85) (width 0.25) (layer "F.Cu") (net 2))
 (segment (start 116.33 53.85) (end 116.33 52.07) (width 0.25) (layer "F.Cu") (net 2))
 (segment (start 138.43 63.5) (end 138.43 71.21) (width 0.25) (layer "F.Cu") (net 2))
 (segment (start 137.16 58.42) (end 130.81 52.07) (width 0.25) (layer "F.Cu") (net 2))
 (segment (start 124.83 87.31) (end 124.97 87.45) (width 0.25) (layer "F.Cu") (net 2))
 (segment (start 102.87 76.2) (end 102.87 68.4) (width 0.25) (layer "F.Cu") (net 2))
 (segment (start 104.14 77.29) (end 103.96 77.29) (width 0.25) (layer "F.Cu") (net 2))
 (segment (start 135.89 73.66) (end 135.89 80.01) (width 0.25) (layer "F.Cu") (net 2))
 (segment (start 131.13 84.77) (end 130.81 84.77) (width 0.25) (layer "F.Cu") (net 2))
 (segment (start 135.89 80.01) (end 131.13 84.77) (width 0.25) (layer "F.Cu") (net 2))
 (segment (start 104.14 81.28) (end 110.49 87.63) (width 0.25) (layer "F.Cu") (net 2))
 (segment (start 105.41 64.77) (end 104.14 66.04) (width 0.25) (layer "F.Cu") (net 2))
 (segment (start 137.16 62.41) (end 137.34 62.41) (width 0.25) (layer "F.Cu") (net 2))
 (segment (start 104.14 77.29) (end 104.14 81.28) (width 0.25) (layer "F.Cu") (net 2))
 (segment (start 128.65 52.07) (end 130.81 52.07) (width 0.25) (layer "F.Cu") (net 2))
 (segment (start 137.07 72.48) (end 135.89 73.66) (width 0.25) (layer "F.Cu") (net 2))
 (segment (start 105.41 59.69) (end 105.41 64.77) (width 0.25) (layer "F.Cu") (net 2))
 (segment (start 130.63 56.97) (end 133.86 60.2) (width 0.25) (layer "F.Cu") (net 49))
 (segment (start 133.86 60.2) (end 133.86 62.41) (width 0.25) (layer "F.Cu") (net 49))
 (segment (start 128.65 56.97) (end 130.63 56.97) (width 0.25) (layer "F.Cu") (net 49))
 (segment (start 137.16 67.31) (end 137.16 68.58) (width 0.25) (layer "F.Cu") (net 50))
 (segment (start 137.16 68.58) (end 133.86 71.88) (width 0.25) (layer "F.Cu") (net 50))
 (segment (start 133.86 71.88) (end 133.86 72.48) (width 0.25) (layer "F.Cu") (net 50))
 (segment (start 137.16 81.28) (end 130.99 87.45) (width 0.25) (layer "F.Cu") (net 9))
 (segment (start 137.16 77.38) (end 137.16 81.28) (width 0.25) (layer "F.Cu") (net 9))
 (segment (start 130.99 87.45) (end 128.27 87.45) (width 0.25) (layer "F.Cu") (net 9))
 (segment (start 123.2349 82.55) (end 124.97 82.55) (width 0.25) (layer "F.Cu") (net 6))
 (segment (start 116.33 87.63) (end 118.1549 87.63) (width 0.25) (layer "F.Cu") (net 6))
 (segment (start 118.1549 87.63) (end 123.2349 82.55) (width 0.25) (layer "F.Cu") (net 6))
 (segment (start 110.67 82.73) (end 113.03 82.73) (width 0.25) (layer "F.Cu") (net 5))
 (segment (start 107.44 77.29) (end 107.44 79.5) (width 0.25) (layer "F.Cu") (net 5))
 (segment (start 107.44 79.5) (end 110.67 82.73) (width 0.25) (layer "F.Cu") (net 5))
 (segment (start 107.44 67.82) (end 107.44 67.13) (width 0.25) (layer "F.Cu") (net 4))
 (segment (start 104.14 71.12) (end 107.44 67.82) (width 0.25) (layer "F.Cu") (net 4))
 (segment (start 104.14 72.39) (end 104.14 71.12) (width 0.25) (layer "F.Cu") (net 4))
 (segment (start 104.14 62.23) (end 104.14 58.42) (width 0.25) (layer "F.Cu") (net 3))
 (segment (start 113.03 52.07) (end 110.49 52.07) (width 0.25) (layer "F.Cu") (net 3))
 (segment (start 110.49 52.07) (end 104.14 58.42) (width 0.25) (layer "F.Cu") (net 3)))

